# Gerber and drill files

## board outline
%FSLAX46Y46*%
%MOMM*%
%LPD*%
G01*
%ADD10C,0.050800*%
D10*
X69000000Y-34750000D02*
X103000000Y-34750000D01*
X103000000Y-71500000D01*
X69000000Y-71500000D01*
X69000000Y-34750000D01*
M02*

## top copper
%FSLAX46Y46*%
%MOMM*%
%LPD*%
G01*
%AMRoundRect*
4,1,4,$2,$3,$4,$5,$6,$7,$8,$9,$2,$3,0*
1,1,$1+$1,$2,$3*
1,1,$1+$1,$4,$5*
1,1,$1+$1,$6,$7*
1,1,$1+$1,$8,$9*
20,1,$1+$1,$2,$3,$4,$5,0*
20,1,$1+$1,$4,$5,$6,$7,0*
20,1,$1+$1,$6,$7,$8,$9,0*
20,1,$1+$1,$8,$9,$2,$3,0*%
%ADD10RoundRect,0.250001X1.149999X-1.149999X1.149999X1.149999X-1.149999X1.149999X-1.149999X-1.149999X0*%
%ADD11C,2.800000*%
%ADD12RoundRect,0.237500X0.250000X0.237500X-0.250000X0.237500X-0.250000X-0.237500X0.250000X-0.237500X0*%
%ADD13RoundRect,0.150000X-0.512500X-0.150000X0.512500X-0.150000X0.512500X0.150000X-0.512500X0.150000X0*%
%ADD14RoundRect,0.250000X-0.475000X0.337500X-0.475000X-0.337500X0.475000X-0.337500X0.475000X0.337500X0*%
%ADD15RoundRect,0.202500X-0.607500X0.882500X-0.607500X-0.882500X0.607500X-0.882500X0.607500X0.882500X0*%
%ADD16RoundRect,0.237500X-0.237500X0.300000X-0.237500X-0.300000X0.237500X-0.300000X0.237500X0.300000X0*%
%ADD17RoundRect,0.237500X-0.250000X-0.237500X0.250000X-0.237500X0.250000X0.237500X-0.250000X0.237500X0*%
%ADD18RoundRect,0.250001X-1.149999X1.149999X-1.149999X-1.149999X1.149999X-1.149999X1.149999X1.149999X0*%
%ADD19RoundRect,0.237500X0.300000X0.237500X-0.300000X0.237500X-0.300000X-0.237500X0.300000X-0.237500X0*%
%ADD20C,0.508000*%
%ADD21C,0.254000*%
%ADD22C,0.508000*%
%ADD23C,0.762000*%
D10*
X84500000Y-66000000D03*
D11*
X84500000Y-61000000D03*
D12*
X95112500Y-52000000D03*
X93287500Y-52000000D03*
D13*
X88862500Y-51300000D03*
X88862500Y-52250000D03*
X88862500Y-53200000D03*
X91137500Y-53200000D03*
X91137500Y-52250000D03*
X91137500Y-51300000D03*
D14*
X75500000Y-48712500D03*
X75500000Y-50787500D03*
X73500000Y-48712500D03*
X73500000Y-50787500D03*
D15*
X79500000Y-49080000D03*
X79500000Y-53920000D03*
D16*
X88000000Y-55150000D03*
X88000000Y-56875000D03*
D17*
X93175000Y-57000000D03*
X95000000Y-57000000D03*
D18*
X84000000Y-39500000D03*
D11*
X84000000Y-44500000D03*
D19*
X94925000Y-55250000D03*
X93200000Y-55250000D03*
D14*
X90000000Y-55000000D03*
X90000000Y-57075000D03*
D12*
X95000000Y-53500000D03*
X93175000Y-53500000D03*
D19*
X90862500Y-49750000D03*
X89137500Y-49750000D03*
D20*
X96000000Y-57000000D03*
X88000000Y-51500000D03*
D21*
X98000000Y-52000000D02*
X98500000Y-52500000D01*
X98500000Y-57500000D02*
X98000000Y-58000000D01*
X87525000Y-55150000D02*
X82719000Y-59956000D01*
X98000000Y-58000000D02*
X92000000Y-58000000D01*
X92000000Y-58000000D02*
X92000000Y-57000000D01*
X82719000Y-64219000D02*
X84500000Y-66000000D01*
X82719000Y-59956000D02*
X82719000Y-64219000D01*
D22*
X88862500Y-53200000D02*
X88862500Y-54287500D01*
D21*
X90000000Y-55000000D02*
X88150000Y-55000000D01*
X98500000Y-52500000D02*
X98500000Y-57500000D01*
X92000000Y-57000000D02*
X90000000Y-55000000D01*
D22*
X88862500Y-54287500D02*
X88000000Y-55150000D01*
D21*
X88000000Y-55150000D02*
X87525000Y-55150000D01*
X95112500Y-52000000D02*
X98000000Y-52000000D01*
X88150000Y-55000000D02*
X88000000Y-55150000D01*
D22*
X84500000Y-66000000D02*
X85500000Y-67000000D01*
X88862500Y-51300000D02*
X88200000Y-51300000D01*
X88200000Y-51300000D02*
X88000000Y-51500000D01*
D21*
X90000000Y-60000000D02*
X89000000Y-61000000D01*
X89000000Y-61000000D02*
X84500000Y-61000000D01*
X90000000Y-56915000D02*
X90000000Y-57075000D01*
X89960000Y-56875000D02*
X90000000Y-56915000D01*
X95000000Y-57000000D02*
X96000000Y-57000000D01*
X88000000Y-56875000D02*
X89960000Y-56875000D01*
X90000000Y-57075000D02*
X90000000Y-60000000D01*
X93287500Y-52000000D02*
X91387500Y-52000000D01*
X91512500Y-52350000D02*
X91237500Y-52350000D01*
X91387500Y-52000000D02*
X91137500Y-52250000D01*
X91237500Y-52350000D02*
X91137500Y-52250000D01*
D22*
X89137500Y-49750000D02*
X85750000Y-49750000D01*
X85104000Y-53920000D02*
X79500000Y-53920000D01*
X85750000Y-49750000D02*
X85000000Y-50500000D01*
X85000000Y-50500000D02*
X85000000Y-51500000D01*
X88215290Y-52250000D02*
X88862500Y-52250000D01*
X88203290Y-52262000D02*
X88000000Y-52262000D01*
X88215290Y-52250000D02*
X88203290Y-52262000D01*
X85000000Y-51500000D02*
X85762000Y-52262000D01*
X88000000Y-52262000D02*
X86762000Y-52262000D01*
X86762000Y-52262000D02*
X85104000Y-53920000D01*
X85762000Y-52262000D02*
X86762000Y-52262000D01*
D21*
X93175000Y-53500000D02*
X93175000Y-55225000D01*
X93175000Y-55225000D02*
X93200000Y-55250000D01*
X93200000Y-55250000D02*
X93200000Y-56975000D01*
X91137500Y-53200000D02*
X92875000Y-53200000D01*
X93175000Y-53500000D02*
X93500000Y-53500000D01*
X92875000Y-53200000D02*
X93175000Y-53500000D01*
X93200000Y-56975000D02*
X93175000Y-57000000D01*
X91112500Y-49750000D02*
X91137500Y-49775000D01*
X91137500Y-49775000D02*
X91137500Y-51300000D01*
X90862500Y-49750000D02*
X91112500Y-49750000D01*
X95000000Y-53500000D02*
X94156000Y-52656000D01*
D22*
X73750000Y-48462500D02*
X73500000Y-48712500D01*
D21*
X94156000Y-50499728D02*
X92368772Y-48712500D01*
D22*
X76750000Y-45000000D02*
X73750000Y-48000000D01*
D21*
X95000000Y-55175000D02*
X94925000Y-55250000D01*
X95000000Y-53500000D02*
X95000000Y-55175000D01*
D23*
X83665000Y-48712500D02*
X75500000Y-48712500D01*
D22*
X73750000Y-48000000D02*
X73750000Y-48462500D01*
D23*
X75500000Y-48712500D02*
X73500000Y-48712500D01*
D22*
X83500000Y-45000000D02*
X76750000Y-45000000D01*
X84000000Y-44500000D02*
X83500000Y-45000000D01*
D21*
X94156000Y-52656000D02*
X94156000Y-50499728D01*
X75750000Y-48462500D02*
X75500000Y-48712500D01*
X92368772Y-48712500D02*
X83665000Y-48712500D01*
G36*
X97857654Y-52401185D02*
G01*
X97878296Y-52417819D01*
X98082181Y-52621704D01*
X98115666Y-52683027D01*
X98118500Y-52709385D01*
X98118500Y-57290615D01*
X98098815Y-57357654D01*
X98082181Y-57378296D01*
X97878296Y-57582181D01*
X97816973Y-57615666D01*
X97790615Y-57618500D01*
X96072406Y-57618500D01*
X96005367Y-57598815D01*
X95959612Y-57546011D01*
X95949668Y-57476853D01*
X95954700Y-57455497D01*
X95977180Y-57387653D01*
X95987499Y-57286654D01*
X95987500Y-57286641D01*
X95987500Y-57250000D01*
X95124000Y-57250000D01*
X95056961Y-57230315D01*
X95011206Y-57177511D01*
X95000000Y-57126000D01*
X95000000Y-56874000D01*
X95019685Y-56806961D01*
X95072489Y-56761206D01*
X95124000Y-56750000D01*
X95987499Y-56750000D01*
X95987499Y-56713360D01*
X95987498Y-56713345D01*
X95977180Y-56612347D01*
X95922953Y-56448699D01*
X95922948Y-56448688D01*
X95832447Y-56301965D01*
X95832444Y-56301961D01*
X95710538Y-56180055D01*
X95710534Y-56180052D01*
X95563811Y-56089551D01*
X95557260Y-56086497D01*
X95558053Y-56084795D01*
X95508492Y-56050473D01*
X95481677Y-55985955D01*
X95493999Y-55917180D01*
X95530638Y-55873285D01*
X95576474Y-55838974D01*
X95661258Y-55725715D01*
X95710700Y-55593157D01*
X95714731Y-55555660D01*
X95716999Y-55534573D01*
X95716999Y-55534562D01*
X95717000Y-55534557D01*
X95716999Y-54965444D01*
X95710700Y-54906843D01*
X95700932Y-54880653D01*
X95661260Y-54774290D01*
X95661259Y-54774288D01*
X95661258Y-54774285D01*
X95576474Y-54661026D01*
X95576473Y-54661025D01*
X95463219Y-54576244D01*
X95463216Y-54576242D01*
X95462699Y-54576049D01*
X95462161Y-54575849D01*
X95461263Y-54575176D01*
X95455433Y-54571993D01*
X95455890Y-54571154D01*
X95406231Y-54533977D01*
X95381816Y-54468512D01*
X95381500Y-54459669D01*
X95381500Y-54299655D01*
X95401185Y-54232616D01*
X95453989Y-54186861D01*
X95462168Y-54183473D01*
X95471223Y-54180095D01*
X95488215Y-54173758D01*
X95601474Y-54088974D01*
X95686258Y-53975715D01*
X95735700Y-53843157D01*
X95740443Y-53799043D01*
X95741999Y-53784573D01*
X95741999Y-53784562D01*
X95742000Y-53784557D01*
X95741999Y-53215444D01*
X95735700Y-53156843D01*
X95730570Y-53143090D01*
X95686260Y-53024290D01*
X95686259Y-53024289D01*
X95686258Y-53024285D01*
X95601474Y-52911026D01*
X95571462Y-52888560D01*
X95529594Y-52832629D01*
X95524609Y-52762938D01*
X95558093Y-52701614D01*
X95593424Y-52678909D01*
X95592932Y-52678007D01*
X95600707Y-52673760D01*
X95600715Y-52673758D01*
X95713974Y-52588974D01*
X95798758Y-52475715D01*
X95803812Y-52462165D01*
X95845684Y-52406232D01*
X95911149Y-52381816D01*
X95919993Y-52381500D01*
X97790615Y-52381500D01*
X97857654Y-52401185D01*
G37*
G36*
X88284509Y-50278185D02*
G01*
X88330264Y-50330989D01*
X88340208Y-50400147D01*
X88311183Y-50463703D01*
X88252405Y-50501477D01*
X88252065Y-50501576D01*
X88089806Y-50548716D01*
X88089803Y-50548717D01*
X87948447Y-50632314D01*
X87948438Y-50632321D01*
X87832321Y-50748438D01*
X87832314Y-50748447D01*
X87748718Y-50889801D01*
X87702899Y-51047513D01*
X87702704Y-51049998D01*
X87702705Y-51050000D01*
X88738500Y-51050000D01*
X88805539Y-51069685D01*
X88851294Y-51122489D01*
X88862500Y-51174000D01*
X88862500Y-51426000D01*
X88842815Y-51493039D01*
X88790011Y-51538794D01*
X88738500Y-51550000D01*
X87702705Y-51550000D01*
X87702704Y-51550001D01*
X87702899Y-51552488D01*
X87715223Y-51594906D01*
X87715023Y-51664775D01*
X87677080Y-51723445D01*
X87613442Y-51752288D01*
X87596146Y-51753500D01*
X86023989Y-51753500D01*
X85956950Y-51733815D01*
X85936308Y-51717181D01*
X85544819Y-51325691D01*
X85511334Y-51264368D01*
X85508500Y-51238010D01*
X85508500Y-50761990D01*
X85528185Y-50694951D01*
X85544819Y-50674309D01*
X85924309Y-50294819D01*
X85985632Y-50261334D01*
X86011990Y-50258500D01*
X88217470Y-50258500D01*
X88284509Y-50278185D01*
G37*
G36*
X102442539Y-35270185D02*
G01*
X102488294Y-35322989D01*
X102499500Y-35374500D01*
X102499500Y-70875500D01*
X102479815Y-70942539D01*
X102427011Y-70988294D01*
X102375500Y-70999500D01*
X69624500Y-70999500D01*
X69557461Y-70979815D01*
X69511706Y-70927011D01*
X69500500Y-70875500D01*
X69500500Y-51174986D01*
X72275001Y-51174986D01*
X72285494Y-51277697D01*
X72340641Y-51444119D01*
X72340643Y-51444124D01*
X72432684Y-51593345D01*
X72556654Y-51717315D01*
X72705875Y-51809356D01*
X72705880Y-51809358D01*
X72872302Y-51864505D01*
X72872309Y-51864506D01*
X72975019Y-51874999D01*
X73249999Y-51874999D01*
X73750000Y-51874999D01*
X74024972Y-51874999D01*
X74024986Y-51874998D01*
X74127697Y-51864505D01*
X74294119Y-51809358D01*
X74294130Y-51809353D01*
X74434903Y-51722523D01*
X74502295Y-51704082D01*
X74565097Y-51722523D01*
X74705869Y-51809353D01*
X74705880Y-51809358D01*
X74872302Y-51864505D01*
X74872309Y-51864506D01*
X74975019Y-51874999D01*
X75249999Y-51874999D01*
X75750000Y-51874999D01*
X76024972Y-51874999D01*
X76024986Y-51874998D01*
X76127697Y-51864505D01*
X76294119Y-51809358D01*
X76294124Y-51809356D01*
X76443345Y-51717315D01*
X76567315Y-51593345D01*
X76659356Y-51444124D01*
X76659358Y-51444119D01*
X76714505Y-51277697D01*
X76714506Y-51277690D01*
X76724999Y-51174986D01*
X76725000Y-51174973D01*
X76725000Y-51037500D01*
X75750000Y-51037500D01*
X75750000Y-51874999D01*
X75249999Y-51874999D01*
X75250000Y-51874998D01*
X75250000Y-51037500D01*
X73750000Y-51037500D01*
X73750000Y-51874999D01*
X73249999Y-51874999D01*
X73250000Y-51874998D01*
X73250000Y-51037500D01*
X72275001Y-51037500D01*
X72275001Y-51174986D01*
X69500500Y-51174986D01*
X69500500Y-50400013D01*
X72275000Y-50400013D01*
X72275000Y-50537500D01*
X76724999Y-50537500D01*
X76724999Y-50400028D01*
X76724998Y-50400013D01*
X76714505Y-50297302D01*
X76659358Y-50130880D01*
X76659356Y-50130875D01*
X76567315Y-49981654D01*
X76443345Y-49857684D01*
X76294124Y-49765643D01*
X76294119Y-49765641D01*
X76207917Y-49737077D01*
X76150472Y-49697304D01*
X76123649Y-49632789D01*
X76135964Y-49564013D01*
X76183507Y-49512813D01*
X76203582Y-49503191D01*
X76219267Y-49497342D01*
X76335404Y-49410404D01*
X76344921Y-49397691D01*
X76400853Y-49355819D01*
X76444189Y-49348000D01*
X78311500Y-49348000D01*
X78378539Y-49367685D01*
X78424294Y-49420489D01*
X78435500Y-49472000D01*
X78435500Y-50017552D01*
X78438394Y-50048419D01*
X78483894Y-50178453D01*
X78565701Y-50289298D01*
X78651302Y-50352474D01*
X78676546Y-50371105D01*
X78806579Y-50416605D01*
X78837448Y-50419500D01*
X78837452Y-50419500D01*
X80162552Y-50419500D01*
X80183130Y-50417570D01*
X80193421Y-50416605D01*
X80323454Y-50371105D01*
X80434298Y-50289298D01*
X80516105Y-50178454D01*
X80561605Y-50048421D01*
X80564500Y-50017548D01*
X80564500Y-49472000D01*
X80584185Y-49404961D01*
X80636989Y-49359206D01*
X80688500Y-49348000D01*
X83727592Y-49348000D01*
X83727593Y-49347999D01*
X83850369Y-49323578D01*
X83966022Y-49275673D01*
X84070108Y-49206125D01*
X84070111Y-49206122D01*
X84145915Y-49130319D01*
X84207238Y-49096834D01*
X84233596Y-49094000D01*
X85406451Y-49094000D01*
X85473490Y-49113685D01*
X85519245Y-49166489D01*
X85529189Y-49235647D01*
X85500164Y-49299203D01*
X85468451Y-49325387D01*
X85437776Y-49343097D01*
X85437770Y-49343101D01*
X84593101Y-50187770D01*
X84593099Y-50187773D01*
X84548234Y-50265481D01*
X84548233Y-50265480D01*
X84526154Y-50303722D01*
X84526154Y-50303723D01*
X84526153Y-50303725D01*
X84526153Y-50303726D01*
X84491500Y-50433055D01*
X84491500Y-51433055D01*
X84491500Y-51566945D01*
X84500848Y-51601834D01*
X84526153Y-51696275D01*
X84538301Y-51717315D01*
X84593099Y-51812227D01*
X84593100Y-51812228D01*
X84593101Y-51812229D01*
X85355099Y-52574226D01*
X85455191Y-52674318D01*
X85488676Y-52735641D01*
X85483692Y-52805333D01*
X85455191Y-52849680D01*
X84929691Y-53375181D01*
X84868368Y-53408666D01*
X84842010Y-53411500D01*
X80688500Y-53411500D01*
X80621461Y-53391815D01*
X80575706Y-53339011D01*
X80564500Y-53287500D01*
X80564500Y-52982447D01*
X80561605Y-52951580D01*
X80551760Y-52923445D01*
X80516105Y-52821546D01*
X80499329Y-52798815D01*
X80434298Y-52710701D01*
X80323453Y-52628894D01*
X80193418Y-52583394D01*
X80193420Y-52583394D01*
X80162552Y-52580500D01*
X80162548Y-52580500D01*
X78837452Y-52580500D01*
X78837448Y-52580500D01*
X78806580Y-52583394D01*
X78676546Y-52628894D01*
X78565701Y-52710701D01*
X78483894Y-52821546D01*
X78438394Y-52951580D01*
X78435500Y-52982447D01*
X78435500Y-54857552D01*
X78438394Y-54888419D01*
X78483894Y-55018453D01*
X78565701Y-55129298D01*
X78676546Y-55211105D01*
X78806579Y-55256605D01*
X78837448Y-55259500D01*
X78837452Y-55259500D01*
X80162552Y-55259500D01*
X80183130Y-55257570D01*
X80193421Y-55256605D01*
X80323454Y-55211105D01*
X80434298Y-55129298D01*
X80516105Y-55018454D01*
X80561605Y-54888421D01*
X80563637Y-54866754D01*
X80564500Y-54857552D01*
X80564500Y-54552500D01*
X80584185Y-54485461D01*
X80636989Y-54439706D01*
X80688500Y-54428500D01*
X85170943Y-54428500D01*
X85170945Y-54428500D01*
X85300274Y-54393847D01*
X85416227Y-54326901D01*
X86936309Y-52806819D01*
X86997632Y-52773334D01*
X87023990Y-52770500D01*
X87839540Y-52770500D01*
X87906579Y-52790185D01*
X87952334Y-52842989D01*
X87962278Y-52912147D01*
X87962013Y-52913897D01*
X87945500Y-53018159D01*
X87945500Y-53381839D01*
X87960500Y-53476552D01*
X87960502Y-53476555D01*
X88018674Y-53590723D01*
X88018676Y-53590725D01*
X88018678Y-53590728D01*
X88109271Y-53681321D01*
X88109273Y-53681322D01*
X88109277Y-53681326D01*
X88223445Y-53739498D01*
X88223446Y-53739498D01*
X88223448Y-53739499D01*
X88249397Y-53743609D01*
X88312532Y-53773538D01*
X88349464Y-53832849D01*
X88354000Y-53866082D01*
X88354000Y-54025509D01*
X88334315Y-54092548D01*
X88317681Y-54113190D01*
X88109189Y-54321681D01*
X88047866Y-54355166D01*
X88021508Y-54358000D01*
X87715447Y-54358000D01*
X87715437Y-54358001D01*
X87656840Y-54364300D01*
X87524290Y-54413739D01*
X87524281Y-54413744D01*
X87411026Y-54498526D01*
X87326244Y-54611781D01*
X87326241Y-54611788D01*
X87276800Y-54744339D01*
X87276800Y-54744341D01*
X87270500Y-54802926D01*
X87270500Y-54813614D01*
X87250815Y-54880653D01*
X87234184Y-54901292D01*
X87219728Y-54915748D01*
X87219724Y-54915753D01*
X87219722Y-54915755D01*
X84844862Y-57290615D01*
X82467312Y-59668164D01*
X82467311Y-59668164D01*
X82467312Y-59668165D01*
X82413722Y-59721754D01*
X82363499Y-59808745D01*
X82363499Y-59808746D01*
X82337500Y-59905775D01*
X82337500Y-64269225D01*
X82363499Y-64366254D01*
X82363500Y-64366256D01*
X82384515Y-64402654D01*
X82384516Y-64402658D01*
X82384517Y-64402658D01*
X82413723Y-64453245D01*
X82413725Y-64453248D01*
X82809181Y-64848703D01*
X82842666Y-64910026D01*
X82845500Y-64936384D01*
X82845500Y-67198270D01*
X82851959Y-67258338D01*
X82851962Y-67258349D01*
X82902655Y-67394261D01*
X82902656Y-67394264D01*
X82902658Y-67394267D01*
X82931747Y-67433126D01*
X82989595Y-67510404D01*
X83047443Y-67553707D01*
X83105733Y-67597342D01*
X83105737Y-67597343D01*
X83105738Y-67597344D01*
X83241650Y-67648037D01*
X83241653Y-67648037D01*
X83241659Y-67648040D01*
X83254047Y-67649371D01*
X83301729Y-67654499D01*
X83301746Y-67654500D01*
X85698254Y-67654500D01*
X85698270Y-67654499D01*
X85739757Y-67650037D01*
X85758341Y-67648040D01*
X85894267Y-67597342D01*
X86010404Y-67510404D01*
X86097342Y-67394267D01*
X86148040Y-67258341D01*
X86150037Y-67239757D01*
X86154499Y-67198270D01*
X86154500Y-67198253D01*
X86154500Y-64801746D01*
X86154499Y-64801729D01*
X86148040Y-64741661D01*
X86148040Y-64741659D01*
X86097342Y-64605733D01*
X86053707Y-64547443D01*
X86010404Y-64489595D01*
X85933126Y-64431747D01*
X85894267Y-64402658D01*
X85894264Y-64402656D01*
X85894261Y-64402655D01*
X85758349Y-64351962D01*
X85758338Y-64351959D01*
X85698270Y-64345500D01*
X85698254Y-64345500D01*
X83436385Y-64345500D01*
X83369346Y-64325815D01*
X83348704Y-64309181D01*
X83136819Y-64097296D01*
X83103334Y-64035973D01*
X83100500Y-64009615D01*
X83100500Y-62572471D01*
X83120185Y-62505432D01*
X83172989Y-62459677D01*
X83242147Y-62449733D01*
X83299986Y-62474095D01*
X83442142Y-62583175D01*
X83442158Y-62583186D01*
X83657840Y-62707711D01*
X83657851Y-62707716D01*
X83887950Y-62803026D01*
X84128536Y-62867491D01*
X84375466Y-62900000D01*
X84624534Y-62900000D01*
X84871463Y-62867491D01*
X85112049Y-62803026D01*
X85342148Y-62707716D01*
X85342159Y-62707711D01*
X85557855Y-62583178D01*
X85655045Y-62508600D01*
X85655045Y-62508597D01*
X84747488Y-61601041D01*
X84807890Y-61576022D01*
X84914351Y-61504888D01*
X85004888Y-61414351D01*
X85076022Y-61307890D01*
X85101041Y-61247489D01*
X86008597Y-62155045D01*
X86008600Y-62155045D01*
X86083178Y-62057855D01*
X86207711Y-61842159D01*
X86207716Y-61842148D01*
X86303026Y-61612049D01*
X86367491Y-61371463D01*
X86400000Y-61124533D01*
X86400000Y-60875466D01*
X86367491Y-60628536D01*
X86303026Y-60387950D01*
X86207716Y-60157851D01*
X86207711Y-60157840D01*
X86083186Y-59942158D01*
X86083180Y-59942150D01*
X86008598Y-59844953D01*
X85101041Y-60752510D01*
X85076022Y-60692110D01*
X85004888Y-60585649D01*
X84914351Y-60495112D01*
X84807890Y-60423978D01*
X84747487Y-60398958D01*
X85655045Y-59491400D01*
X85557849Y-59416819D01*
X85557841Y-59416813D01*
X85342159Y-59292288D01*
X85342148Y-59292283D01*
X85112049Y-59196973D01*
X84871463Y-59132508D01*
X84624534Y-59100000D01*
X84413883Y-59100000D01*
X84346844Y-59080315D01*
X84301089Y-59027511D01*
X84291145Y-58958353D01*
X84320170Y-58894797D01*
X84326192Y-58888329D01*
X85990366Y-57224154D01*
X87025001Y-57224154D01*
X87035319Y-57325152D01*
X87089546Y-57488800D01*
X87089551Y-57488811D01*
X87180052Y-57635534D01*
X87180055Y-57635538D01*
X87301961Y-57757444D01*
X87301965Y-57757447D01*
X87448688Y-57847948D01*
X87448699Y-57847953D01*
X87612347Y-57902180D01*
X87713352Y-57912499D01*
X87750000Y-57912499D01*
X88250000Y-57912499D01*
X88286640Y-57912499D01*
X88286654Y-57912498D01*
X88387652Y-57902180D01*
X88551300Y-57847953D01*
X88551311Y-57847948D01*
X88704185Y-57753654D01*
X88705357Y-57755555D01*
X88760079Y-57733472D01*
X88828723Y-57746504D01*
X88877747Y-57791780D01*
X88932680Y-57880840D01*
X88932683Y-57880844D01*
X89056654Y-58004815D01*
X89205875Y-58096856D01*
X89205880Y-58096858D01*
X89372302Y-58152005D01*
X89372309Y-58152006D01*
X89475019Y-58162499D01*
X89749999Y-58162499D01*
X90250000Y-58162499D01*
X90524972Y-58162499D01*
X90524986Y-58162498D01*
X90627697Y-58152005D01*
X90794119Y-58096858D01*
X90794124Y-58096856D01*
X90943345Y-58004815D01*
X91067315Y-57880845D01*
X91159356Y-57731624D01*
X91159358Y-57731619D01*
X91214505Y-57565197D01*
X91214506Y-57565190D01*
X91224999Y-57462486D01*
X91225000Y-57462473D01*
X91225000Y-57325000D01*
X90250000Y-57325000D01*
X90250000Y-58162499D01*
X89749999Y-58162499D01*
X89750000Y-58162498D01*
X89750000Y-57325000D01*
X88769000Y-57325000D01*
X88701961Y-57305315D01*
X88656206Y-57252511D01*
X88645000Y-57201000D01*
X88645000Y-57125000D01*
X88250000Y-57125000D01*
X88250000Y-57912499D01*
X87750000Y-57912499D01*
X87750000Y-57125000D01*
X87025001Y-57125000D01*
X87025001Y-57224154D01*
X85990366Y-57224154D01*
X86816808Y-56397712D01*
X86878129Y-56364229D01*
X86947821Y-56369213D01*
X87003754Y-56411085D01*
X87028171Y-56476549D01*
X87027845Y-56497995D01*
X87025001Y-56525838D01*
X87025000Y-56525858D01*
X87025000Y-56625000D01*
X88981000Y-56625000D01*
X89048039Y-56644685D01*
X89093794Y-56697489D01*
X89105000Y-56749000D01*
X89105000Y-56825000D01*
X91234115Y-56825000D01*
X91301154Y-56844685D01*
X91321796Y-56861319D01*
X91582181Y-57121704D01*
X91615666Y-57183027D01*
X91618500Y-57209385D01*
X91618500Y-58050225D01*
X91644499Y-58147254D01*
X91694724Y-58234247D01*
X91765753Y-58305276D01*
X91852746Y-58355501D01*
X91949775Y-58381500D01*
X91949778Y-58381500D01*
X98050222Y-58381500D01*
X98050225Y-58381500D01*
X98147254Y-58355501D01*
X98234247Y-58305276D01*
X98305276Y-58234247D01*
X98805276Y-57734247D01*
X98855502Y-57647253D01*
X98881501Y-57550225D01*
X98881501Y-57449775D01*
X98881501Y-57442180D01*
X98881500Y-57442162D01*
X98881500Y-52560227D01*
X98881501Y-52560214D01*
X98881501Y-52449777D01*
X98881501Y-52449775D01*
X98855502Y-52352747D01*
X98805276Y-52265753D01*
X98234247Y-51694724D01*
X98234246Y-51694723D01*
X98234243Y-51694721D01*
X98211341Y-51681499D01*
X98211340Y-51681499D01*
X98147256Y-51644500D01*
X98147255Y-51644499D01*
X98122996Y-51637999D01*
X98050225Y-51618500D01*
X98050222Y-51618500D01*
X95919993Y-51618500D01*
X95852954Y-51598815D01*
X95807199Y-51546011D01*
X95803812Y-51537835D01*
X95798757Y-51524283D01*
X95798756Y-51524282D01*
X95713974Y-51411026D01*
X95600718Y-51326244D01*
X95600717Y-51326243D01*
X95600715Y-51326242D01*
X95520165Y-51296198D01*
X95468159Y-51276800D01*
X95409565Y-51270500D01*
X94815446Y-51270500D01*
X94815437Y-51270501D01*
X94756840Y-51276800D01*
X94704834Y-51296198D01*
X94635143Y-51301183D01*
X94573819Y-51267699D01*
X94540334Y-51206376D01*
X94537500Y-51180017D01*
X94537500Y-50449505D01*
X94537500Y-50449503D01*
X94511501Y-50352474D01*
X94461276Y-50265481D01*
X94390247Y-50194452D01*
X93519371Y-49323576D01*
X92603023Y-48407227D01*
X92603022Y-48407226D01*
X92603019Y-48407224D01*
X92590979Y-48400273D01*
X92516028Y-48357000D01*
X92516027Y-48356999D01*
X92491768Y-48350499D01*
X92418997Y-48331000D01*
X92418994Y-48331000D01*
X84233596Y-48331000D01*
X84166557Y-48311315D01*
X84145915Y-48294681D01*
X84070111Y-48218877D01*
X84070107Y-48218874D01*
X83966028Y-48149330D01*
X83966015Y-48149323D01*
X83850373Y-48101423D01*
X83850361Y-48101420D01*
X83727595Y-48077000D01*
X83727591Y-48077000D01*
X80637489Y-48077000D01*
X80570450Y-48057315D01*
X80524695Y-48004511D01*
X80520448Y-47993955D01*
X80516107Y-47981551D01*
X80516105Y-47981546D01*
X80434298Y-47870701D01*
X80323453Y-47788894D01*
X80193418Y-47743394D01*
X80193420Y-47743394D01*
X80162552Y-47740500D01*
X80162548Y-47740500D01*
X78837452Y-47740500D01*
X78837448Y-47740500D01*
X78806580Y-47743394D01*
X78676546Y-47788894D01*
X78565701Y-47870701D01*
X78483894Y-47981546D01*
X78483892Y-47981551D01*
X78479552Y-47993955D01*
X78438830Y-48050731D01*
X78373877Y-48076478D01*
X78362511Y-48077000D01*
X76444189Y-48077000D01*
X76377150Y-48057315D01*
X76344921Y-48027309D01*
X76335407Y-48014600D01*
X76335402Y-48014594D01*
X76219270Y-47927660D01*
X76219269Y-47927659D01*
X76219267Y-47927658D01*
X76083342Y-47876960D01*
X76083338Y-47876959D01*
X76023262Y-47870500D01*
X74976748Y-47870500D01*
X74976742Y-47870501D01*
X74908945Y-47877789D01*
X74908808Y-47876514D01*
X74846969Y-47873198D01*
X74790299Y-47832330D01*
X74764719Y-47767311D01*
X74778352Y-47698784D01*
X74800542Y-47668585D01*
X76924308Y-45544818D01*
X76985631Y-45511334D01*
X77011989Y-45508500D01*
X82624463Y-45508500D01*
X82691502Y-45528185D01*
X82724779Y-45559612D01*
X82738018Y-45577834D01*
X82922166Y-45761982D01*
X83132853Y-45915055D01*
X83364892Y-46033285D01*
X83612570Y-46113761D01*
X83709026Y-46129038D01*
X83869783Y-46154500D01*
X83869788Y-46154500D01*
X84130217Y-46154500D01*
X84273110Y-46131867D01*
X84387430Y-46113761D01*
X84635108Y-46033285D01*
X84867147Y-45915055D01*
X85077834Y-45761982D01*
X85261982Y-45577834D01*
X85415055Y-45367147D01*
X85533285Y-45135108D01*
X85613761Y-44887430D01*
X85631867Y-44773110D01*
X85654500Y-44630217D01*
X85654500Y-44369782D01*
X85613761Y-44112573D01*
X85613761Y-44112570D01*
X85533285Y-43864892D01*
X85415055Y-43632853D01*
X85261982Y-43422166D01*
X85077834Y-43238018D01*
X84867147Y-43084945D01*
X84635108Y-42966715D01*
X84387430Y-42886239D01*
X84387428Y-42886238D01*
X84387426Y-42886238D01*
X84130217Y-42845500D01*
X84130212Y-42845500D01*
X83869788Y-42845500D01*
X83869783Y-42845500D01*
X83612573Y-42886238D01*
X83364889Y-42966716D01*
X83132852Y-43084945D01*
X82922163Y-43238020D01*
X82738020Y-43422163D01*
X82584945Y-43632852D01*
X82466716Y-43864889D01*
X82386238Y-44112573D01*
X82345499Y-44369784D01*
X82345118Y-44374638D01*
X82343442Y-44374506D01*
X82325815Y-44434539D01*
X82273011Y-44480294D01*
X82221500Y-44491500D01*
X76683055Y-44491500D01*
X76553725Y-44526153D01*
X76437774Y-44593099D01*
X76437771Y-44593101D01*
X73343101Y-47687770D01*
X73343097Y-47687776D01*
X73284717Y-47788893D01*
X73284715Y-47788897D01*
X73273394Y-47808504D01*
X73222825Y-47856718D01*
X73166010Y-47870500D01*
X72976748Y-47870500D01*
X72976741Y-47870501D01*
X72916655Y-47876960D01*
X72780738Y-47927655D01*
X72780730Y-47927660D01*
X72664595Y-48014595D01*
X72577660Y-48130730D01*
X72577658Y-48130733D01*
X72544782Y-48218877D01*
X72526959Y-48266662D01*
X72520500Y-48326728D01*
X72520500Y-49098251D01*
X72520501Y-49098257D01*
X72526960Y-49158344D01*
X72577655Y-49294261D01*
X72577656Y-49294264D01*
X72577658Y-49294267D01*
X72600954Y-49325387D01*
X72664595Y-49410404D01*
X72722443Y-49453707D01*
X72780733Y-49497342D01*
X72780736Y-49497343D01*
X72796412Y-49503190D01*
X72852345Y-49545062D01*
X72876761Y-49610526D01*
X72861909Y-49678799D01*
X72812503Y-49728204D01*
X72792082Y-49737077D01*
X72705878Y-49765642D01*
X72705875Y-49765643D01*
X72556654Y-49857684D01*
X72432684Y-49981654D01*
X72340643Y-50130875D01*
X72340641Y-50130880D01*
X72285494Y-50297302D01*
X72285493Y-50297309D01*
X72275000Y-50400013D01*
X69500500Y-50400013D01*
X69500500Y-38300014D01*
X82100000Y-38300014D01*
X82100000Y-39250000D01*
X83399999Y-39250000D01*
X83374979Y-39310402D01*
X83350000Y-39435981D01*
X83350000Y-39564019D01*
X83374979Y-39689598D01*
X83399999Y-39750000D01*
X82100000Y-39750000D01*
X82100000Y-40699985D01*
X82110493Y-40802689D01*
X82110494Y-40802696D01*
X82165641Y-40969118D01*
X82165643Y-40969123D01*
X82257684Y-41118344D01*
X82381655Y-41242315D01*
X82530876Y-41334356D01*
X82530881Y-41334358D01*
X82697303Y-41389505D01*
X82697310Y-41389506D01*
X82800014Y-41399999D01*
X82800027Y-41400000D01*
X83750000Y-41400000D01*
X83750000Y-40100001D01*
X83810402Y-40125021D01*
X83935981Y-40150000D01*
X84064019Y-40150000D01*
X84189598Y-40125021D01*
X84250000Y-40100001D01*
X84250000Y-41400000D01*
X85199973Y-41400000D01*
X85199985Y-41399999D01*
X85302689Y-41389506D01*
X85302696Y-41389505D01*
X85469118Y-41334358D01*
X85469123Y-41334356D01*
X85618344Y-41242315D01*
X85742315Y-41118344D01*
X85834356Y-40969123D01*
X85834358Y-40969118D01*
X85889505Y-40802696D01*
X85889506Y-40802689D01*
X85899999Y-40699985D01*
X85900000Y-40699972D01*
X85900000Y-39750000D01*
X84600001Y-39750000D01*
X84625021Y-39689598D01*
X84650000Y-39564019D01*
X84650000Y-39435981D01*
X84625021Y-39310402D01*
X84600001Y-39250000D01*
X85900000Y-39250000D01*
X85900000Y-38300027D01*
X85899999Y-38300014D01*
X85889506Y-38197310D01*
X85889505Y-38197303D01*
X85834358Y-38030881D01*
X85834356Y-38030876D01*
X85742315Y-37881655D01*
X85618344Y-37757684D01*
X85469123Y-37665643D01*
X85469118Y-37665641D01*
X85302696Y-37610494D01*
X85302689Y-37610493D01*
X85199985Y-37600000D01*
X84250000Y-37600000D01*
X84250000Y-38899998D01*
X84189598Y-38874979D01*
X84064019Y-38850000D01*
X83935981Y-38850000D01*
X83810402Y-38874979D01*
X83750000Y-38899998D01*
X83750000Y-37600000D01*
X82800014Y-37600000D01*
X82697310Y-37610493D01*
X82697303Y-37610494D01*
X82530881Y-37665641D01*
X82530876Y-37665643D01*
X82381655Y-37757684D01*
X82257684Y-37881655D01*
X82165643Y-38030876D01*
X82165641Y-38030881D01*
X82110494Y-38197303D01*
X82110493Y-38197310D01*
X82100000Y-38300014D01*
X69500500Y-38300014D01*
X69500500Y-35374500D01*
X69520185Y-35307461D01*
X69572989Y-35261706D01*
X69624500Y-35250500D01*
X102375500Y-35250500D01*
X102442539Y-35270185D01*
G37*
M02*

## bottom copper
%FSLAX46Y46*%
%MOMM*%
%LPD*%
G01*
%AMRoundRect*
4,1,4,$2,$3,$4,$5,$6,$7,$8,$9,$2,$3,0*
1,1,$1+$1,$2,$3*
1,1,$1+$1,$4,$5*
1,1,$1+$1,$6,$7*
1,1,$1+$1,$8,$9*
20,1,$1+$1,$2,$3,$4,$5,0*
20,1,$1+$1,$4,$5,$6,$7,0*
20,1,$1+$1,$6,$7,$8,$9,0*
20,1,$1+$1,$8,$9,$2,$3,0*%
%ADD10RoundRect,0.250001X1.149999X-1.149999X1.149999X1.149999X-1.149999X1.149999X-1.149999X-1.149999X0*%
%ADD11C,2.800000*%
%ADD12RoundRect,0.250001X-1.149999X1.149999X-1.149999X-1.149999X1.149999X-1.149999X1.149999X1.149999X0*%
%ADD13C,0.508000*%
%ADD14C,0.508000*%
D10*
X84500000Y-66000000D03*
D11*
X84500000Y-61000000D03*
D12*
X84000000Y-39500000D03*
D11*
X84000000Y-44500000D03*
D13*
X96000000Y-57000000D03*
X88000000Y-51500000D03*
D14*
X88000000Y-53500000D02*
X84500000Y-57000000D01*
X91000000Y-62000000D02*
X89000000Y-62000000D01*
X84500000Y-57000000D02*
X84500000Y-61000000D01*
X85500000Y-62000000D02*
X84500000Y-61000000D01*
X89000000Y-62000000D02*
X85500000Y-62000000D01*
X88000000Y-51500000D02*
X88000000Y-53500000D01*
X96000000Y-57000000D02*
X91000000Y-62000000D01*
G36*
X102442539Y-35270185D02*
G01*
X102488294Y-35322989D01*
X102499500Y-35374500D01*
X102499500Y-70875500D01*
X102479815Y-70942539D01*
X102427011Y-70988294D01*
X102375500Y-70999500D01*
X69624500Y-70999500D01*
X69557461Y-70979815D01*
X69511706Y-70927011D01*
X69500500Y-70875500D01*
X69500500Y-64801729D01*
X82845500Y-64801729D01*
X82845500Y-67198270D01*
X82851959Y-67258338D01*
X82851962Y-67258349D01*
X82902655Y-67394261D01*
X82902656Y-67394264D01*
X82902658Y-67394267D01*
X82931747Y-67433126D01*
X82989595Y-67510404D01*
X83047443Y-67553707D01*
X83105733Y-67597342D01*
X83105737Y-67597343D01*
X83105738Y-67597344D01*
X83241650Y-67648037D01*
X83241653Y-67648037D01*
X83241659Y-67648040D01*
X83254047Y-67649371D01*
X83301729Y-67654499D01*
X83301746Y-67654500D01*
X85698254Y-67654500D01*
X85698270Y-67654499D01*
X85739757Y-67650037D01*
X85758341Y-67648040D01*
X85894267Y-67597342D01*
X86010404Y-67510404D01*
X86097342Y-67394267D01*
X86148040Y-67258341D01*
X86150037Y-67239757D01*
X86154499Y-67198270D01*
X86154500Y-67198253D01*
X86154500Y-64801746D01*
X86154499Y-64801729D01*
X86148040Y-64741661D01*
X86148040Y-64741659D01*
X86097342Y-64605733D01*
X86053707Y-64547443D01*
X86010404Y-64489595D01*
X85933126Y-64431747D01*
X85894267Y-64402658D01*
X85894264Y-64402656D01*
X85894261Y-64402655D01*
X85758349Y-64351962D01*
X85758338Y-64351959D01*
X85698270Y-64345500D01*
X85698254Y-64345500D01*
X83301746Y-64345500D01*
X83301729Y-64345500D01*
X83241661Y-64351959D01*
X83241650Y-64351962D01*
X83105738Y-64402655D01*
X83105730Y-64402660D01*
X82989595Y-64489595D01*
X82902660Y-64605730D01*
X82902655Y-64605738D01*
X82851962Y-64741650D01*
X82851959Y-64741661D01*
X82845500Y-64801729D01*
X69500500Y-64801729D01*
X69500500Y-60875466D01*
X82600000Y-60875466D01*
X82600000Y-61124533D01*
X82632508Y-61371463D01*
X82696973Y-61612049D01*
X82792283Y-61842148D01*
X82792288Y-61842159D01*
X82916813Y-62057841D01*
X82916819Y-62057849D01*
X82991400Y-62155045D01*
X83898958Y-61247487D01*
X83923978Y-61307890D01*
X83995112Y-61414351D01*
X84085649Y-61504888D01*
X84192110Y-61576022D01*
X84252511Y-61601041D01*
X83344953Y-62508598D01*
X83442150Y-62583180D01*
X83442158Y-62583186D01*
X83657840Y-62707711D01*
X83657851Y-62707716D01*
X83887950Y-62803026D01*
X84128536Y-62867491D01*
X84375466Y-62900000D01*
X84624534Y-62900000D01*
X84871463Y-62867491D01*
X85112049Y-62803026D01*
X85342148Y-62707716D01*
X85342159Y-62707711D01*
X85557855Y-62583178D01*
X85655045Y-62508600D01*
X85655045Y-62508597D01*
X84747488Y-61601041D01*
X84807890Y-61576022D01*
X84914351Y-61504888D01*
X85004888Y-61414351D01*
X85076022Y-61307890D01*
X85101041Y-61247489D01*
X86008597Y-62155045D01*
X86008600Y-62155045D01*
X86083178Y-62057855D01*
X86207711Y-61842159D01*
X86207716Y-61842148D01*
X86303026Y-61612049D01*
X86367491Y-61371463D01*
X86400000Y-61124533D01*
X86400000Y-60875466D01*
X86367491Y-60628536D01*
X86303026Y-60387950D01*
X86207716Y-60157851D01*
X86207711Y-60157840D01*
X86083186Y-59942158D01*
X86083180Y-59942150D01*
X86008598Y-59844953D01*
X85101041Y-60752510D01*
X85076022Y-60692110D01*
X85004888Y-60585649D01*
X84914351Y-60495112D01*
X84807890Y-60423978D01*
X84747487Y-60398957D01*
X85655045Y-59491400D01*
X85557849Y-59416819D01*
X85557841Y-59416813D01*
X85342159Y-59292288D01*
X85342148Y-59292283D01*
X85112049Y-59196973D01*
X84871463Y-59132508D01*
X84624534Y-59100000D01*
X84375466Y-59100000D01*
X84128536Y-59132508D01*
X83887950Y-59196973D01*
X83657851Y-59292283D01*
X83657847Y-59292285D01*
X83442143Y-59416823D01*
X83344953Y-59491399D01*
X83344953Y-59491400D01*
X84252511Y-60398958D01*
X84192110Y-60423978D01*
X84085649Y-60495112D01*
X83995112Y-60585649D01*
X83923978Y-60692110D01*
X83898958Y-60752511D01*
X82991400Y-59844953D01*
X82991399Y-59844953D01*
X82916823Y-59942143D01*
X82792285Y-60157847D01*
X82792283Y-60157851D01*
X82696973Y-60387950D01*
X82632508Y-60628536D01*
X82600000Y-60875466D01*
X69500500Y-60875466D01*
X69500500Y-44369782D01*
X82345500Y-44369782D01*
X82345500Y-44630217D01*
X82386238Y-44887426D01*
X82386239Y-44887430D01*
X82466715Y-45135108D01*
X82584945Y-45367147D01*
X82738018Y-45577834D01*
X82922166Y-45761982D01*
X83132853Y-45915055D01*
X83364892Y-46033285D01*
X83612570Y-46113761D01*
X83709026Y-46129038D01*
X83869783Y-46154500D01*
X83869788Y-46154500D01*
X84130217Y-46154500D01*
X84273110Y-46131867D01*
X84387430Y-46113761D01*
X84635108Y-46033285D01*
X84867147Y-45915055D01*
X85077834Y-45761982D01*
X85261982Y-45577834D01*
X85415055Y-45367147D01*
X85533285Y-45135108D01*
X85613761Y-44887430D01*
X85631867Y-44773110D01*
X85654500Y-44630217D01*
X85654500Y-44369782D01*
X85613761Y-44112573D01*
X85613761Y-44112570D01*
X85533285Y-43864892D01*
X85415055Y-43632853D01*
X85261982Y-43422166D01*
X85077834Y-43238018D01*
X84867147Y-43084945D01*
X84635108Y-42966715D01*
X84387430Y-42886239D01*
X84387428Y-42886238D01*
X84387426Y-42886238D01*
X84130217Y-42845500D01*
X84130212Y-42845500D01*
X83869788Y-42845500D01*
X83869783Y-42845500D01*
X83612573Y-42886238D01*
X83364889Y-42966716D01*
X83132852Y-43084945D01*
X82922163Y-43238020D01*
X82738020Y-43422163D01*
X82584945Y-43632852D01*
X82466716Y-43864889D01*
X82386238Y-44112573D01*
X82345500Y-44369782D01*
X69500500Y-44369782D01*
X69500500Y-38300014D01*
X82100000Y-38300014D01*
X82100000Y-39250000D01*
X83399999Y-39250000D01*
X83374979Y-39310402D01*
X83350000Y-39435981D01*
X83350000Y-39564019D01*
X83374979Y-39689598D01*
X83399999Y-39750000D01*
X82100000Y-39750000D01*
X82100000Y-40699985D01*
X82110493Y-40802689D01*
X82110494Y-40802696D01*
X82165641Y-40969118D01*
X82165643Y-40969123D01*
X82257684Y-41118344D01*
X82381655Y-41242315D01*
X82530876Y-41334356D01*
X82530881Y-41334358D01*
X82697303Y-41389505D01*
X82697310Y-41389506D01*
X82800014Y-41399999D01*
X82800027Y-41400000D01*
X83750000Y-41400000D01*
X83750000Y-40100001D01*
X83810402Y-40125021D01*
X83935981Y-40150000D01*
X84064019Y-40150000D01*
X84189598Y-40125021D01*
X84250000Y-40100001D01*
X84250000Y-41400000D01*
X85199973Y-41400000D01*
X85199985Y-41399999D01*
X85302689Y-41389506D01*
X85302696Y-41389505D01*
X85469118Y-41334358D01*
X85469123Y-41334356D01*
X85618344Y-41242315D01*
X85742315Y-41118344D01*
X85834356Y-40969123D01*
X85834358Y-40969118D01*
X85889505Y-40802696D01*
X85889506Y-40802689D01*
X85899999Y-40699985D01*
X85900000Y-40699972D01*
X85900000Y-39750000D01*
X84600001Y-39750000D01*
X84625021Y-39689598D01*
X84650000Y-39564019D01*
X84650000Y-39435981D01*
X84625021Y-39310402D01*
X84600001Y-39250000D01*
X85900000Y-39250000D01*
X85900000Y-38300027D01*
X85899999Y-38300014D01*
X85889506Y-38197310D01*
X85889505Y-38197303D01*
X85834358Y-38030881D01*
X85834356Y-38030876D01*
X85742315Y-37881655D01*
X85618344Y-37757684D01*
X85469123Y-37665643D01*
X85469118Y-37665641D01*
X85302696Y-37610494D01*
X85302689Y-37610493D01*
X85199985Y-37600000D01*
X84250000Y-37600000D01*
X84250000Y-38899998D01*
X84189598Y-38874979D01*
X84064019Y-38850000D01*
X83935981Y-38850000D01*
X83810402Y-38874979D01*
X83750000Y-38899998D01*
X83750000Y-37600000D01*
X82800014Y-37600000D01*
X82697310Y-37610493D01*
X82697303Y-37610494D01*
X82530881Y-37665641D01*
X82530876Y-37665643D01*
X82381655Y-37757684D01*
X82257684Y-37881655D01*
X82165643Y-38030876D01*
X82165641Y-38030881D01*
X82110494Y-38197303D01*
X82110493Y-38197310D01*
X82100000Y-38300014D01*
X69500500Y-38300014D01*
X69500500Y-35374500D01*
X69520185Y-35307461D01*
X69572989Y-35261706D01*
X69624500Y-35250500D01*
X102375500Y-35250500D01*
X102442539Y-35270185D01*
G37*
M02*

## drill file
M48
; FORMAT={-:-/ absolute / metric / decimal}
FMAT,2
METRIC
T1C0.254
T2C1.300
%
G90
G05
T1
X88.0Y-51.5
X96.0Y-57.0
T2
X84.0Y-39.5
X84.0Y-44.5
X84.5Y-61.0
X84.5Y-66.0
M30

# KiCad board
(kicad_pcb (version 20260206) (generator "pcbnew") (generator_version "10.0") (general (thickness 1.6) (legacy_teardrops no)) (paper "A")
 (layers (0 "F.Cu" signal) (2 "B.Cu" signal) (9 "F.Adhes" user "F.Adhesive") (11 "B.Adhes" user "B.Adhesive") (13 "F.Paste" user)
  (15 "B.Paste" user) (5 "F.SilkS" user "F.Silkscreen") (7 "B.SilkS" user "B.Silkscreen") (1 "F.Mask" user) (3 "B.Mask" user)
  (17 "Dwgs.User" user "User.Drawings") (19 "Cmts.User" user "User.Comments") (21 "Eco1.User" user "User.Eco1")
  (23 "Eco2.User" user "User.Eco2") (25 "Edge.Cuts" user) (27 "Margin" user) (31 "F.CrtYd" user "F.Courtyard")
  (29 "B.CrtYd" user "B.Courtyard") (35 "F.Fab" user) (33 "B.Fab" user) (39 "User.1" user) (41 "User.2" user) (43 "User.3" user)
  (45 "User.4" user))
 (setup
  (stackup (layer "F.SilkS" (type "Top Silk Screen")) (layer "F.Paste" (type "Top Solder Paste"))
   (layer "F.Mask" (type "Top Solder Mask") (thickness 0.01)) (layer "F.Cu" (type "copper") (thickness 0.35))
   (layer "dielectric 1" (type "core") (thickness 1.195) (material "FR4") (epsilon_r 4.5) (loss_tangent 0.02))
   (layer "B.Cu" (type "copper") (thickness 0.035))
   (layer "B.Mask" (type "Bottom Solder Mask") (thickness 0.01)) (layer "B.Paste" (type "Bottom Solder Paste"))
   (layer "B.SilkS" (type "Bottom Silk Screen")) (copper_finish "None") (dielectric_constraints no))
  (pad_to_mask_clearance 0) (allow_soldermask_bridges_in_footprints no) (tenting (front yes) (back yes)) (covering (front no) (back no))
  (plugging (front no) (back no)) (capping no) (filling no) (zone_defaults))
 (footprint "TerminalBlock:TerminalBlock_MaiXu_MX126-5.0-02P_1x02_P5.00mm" (layer "F.Cu") (at 84.5 66 90)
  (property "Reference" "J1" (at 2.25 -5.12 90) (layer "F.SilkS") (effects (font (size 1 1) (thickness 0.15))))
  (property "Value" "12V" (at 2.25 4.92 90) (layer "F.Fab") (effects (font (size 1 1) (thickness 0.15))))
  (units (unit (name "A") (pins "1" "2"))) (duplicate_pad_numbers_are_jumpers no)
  (pad "1" thru_hole roundrect (at 0 0 90) (size 2.8 2.8) (drill 1.3) (layers "*.Cu" "*.Mask") (remove_unused_layers no)
   (roundrect_rratio 0.089286) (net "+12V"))
  (pad "2" thru_hole circle (at 5 0 90) (size 2.8 2.8) (drill 1.3) (layers "*.Cu" "*.Mask") (remove_unused_layers no) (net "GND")))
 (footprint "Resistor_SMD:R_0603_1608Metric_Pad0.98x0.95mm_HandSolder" (layer "F.Cu") (at 94.2 52 180)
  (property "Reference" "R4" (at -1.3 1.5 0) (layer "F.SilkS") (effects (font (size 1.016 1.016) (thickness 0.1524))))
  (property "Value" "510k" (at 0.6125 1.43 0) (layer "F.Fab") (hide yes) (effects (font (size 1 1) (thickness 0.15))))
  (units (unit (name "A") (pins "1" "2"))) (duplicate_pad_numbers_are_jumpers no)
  (pad "1" smd roundrect (at -0.9125 0 180) (size 0.975 0.95) (layers "F.Cu" "F.Mask" "F.Paste") (roundrect_rratio 0.25) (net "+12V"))
  (pad "2" smd roundrect (at 0.9125 0 180) (size 0.975 0.95) (layers "F.Cu" "F.Mask" "F.Paste") (roundrect_rratio 0.25) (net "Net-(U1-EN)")))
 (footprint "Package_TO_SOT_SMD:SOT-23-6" (layer "F.Cu") (at 90 52.25)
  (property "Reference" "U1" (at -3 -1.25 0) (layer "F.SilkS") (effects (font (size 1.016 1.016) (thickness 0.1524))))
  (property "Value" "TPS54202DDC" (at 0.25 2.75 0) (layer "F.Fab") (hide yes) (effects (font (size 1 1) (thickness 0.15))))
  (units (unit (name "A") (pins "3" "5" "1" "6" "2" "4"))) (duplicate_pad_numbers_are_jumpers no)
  (pad "1" smd roundrect (at -1.1375 -0.95) (size 1.325 0.6) (layers "F.Cu" "F.Mask" "F.Paste") (roundrect_rratio 0.25) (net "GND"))
  (pad "2" smd roundrect (at -1.1375 0) (size 1.325 0.6) (layers "F.Cu" "F.Mask" "F.Paste") (roundrect_rratio 0.25) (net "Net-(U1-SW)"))
  (pad "3" smd roundrect (at -1.1375 0.95) (size 1.325 0.6) (layers "F.Cu" "F.Mask" "F.Paste") (roundrect_rratio 0.25) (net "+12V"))
  (pad "4" smd roundrect (at 1.1375 0.95) (size 1.325 0.6) (layers "F.Cu" "F.Mask" "F.Paste") (roundrect_rratio 0.25) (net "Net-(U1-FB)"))
  (pad "5" smd roundrect (at 1.1375 0) (size 1.325 0.6) (layers "F.Cu" "F.Mask" "F.Paste") (roundrect_rratio 0.25) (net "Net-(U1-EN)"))
  (pad "6" smd roundrect (at 1.1375 -0.95) (size 1.325 0.6) (layers "F.Cu" "F.Mask" "F.Paste") (roundrect_rratio 0.25) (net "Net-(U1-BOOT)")))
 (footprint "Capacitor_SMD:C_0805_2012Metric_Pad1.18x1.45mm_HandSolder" (layer "F.Cu") (at 75.5 49.75 -90)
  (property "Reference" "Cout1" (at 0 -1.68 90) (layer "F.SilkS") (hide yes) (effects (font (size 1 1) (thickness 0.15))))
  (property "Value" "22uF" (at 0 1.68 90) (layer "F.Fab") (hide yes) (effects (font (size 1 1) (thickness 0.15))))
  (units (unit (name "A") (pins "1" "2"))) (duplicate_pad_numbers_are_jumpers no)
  (pad "1" smd roundrect (at -1.0375 0 270) (size 1.175 1.45) (layers "F.Cu" "F.Mask" "F.Paste") (roundrect_rratio 0.212766) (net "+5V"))
  (pad "2" smd roundrect (at 1.0375 0 270) (size 1.175 1.45) (layers "F.Cu" "F.Mask" "F.Paste") (roundrect_rratio 0.212766) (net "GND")))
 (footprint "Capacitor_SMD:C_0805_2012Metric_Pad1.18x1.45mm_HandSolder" (layer "F.Cu") (at 73.5 49.75 -90)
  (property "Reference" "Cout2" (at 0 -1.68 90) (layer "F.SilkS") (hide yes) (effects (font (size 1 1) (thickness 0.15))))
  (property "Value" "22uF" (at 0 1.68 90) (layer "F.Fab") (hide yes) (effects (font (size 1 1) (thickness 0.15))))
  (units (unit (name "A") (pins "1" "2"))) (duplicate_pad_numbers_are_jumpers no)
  (pad "1" smd roundrect (at -1.0375 0 270) (size 1.175 1.45) (layers "F.Cu" "F.Mask" "F.Paste") (roundrect_rratio 0.212766) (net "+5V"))
  (pad "2" smd roundrect (at 1.0375 0 270) (size 1.175 1.45) (layers "F.Cu" "F.Mask" "F.Paste") (roundrect_rratio 0.212766) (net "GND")))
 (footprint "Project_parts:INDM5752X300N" (layer "F.Cu") (at 79.5 51.5 -90)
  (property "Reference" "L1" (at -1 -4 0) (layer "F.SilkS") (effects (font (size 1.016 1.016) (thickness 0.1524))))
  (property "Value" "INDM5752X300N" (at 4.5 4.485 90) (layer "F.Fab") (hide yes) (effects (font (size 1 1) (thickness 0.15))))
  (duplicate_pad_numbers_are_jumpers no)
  (pad "1" smd roundrect (at -2.42 0 270) (size 2.17 1.62) (layers "F.Cu" "F.Mask" "F.Paste") (roundrect_rratio 0.125) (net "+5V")
   (solder_mask_margin 0.102))
  (pad "2" smd roundrect (at 2.42 0 270) (size 2.17 1.62) (layers "F.Cu" "F.Mask" "F.Paste") (roundrect_rratio 0.125) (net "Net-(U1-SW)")
   (solder_mask_margin 0.102)))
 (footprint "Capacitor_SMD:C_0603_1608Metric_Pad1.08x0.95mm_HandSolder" (layer "F.Cu") (at 88 56.0125 -90)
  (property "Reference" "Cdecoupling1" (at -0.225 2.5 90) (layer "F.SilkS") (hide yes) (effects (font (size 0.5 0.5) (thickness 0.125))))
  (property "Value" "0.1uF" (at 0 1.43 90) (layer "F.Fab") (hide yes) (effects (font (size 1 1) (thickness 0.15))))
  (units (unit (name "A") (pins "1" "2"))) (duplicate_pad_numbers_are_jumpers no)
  (pad "1" smd roundrect (at -0.8625 0 270) (size 1.075 0.95) (layers "F.Cu" "F.Mask" "F.Paste") (roundrect_rratio 0.25) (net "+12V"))
  (pad "2" smd roundrect (at 0.8625 0 270) (size 1.075 0.95) (layers "F.Cu" "F.Mask" "F.Paste") (roundrect_rratio 0.25) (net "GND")))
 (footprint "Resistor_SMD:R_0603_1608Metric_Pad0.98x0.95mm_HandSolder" (layer "F.Cu") (at 94.0875 57)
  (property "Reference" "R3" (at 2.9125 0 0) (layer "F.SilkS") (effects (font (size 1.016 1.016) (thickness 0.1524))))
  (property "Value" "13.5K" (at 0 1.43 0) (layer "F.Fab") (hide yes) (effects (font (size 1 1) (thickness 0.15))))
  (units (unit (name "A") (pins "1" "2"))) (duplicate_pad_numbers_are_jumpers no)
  (pad "1" smd roundrect (at -0.9125 0) (size 0.975 0.95) (layers "F.Cu" "F.Mask" "F.Paste") (roundrect_rratio 0.25) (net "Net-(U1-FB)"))
  (pad "2" smd roundrect (at 0.9125 0) (size 0.975 0.95) (layers "F.Cu" "F.Mask" "F.Paste") (roundrect_rratio 0.25) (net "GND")))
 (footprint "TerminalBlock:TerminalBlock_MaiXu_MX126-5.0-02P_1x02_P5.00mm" (layer "F.Cu") (at 84 39.5 -90)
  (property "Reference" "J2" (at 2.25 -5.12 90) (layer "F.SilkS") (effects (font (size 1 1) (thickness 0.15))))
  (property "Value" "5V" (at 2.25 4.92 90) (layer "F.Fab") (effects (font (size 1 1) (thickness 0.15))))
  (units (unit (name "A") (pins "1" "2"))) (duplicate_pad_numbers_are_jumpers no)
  (pad "1" thru_hole roundrect (at 0 0 270) (size 2.8 2.8) (drill 1.3) (layers "*.Cu" "*.Mask") (remove_unused_layers no)
   (roundrect_rratio 0.089286) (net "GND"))
  (pad "2" thru_hole circle (at 5 0 270) (size 2.8 2.8) (drill 1.3) (layers "*.Cu" "*.Mask") (remove_unused_layers no) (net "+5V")))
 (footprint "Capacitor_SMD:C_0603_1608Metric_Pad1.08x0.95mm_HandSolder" (layer "F.Cu") (at 94.0625 55.25 180)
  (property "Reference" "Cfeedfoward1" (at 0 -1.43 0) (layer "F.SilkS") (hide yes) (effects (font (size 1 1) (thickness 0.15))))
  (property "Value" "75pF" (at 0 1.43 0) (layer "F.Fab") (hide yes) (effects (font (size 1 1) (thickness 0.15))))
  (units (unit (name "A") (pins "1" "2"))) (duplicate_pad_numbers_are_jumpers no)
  (pad "1" smd roundrect (at -0.8625 0 180) (size 1.075 0.95) (layers "F.Cu" "F.Mask" "F.Paste") (roundrect_rratio 0.25) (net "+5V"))
  (pad "2" smd roundrect (at 0.8625 0 180) (size 1.075 0.95) (layers "F.Cu" "F.Mask" "F.Paste") (roundrect_rratio 0.25) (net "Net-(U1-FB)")))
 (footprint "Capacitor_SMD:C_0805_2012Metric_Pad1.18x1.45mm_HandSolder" (layer "F.Cu") (at 90 56.0375 -90)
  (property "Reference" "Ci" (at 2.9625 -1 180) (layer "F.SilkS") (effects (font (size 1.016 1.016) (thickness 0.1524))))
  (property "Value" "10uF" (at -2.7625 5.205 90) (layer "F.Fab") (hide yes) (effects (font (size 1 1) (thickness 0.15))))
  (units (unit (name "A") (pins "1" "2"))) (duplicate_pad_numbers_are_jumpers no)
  (pad "1" smd roundrect (at -1.0375 0 270) (size 1.175 1.45) (layers "F.Cu" "F.Mask" "F.Paste") (roundrect_rratio 0.212766) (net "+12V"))
  (pad "2" smd roundrect (at 1.0375 0 270) (size 1.175 1.45) (layers "F.Cu" "F.Mask" "F.Paste") (roundrect_rratio 0.212766) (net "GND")))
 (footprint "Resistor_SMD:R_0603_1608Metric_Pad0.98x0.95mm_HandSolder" (layer "F.Cu") (at 94.0875 53.5 180)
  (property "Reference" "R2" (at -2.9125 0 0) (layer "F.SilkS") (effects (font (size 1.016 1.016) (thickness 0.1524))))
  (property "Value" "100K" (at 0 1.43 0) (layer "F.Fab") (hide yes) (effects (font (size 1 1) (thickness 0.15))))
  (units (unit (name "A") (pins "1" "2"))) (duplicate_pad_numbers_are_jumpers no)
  (pad "1" smd roundrect (at -0.9125 0 180) (size 0.975 0.95) (layers "F.Cu" "F.Mask" "F.Paste") (roundrect_rratio 0.25) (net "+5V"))
  (pad "2" smd roundrect (at 0.9125 0 180) (size 0.975 0.95) (layers "F.Cu" "F.Mask" "F.Paste") (roundrect_rratio 0.25) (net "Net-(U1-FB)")))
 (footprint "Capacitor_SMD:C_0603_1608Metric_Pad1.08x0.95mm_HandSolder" (layer "F.Cu") (at 90 49.75 180)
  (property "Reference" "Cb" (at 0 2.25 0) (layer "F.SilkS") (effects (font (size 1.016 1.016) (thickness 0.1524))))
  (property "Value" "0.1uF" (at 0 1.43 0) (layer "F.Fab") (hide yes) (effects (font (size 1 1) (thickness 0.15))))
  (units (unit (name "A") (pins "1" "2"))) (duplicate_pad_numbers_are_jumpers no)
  (pad "1" smd roundrect (at -0.8625 0 180) (size 1.075 0.95) (layers "F.Cu" "F.Mask" "F.Paste") (roundrect_rratio 0.25)
   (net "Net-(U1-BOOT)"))
  (pad "2" smd roundrect (at 0.8625 0 180) (size 1.075 0.95) (layers "F.Cu" "F.Mask" "F.Paste") (roundrect_rratio 0.25) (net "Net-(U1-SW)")))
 (gr_rect (start 69 34.75) (end 103 71.5) (stroke (width 0.0508) (type default)) (fill no) (layer "Edge.Cuts"))
 (segment (start 98 52) (end 98.5 52.5) (width 0.254) (layer "F.Cu") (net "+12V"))
 (segment (start 98.5 57.5) (end 98 58) (width 0.254) (layer "F.Cu") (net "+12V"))
 (segment (start 87.525 55.15) (end 82.719 59.956) (width 0.254) (layer "F.Cu") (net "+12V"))
 (segment (start 98 58) (end 92 58) (width 0.254) (layer "F.Cu") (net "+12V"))
 (segment (start 92 58) (end 92 57) (width 0.254) (layer "F.Cu") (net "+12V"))
 (segment (start 82.719 64.219) (end 84.5 66) (width 0.254) (layer "F.Cu") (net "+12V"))
 (segment (start 82.719 59.956) (end 82.719 64.219) (width 0.254) (layer "F.Cu") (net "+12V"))
 (segment (start 88.8625 53.2) (end 88.8625 54.2875) (width 0.508) (layer "F.Cu") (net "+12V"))
 (segment (start 90 55) (end 88.15 55) (width 0.254) (layer "F.Cu") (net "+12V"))
 (segment (start 98.5 52.5) (end 98.5 57.5) (width 0.254) (layer "F.Cu") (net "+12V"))
 (segment (start 92 57) (end 90 55) (width 0.254) (layer "F.Cu") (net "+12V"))
 (segment (start 88.8625 54.2875) (end 88 55.15) (width 0.508) (layer "F.Cu") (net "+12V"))
 (segment (start 88 55.15) (end 87.525 55.15) (width 0.254) (layer "F.Cu") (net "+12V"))
 (segment (start 95.1125 52) (end 98 52) (width 0.254) (layer "F.Cu") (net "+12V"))
 (segment (start 88.15 55) (end 88 55.15) (width 0.254) (layer "F.Cu") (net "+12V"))
 (segment (start 84.5 66) (end 85.5 67) (width 0.508) (layer "F.Cu") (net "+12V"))
 (segment (start 88.8625 51.3) (end 88.2 51.3) (width 0.508) (layer "F.Cu") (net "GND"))
 (segment (start 88.2 51.3) (end 88 51.5) (width 0.508) (layer "F.Cu") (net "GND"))
 (segment (start 90 60) (end 89 61) (width 0.254) (layer "F.Cu") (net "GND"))
 (segment (start 89 61) (end 84.5 61) (width 0.254) (layer "F.Cu") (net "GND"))
 (segment (start 90 56.915) (end 90 57.075) (width 0.254) (layer "F.Cu") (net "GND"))
 (segment (start 89.96 56.875) (end 90 56.915) (width 0.254) (layer "F.Cu") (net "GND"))
 (segment (start 95 57) (end 96 57) (width 0.254) (layer "F.Cu") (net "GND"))
 (segment (start 88 56.875) (end 89.96 56.875) (width 0.254) (layer "F.Cu") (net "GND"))
 (segment (start 90 57.075) (end 90 60) (width 0.254) (layer "F.Cu") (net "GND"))
 (via (at 96 57) (size 0.508) (drill 0.254) (layers "F.Cu" "B.Cu") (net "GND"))
 (via (at 88 51.5) (size 0.508) (drill 0.254) (layers "F.Cu" "B.Cu") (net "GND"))
 (segment (start 88 53.5) (end 84.5 57) (width 0.508) (layer "B.Cu") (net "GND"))
 (segment (start 91 62) (end 89 62) (width 0.508) (layer "B.Cu") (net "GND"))
 (segment (start 84.5 57) (end 84.5 61) (width 0.508) (layer "B.Cu") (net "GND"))
 (segment (start 85.5 62) (end 84.5 61) (width 0.508) (layer "B.Cu") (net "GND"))
 (segment (start 89 62) (end 85.5 62) (width 0.508) (layer "B.Cu") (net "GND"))
 (segment (start 88 51.5) (end 88 53.5) (width 0.508) (layer "B.Cu") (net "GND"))
 (segment (start 96 57) (end 91 62) (width 0.508) (layer "B.Cu") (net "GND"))
 (segment (start 93.2875 52) (end 91.3875 52) (width 0.254) (layer "F.Cu") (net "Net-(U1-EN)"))
 (segment (start 91.5125 52.35) (end 91.2375 52.35) (width 0.254) (layer "F.Cu") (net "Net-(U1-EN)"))
 (segment (start 91.3875 52) (end 91.1375 52.25) (width 0.254) (layer "F.Cu") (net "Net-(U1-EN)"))
 (segment (start 91.2375 52.35) (end 91.1375 52.25) (width 0.254) (layer "F.Cu") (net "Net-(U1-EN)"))
 (segment (start 89.1375 49.75) (end 85.75 49.75) (width 0.508) (layer "F.Cu") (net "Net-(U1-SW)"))
 (segment (start 85.104 53.92) (end 79.5 53.92) (width 0.508) (layer "F.Cu") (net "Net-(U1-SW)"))
 (segment (start 85.75 49.75) (end 85 50.5) (width 0.508) (layer "F.Cu") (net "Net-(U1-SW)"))
 (segment (start 85 50.5) (end 85 51.5) (width 0.508) (layer "F.Cu") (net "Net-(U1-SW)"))
 (segment (start 88.21529 52.25) (end 88.8625 52.25) (width 0.508) (layer "F.Cu") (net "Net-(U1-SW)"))
 (segment (start 88.20329 52.262) (end 88 52.262) (width 0.508) (layer "F.Cu") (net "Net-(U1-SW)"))
 (segment (start 88.21529 52.25) (end 88.20329 52.262) (width 0.508) (layer "F.Cu") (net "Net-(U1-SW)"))
 (segment (start 85 51.5) (end 85.762 52.262) (width 0.508) (layer "F.Cu") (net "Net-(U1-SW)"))
 (segment (start 88 52.262) (end 86.762 52.262) (width 0.508) (layer "F.Cu") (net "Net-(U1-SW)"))
 (segment (start 86.762 52.262) (end 85.104 53.92) (width 0.508) (layer "F.Cu") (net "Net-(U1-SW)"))
 (segment (start 85.762 52.262) (end 86.762 52.262) (width 0.508) (layer "F.Cu") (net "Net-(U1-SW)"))
 (segment (start 93.175 53.5) (end 93.175 55.225) (width 0.254) (layer "F.Cu") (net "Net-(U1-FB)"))
 (segment (start 93.175 55.225) (end 93.2 55.25) (width 0.254) (layer "F.Cu") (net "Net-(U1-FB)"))
 (segment (start 93.2 55.25) (end 93.2 56.975) (width 0.254) (layer "F.Cu") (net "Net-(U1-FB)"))
 (segment (start 91.1375 53.2) (end 92.875 53.2) (width 0.254) (layer "F.Cu") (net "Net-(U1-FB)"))
 (segment (start 93.175 53.5) (end 93.5 53.5) (width 0.254) (layer "F.Cu") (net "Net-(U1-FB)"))
 (segment (start 92.875 53.2) (end 93.175 53.5) (width 0.254) (layer "F.Cu") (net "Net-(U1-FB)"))
 (segment (start 93.2 56.975) (end 93.175 57) (width 0.254) (layer "F.Cu") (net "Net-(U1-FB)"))
 (segment (start 91.1125 49.75) (end 91.1375 49.775) (width 0.254) (layer "F.Cu") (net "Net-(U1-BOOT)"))
 (segment (start 91.1375 49.775) (end 91.1375 51.3) (width 0.254) (layer "F.Cu") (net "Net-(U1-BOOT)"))
 (segment (start 90.8625 49.75) (end 91.1125 49.75) (width 0.254) (layer "F.Cu") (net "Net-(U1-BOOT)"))
 (segment (start 95 53.5) (end 94.156 52.656) (width 0.254) (layer "F.Cu") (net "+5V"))
 (segment (start 73.75 48.4625) (end 73.5 48.7125) (width 0.508) (layer "F.Cu") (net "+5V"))
 (segment (start 94.156 50.499728) (end 92.368772 48.7125) (width 0.254) (layer "F.Cu") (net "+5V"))
 (segment (start 76.75 45) (end 73.75 48) (width 0.508) (layer "F.Cu") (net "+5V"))
 (segment (start 95 55.175) (end 94.925 55.25) (width 0.254) (layer "F.Cu") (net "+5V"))
 (segment (start 95 53.5) (end 95 55.175) (width 0.254) (layer "F.Cu") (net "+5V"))
 (segment (start 83.665 48.7125) (end 75.5 48.7125) (width 0.762) (layer "F.Cu") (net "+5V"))
 (segment (start 73.75 48) (end 73.75 48.4625) (width 0.508) (layer "F.Cu") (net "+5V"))
 (segment (start 75.5 48.7125) (end 73.5 48.7125) (width 0.762) (layer "F.Cu") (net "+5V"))
 (segment (start 83.5 45) (end 76.75 45) (width 0.508) (layer "F.Cu") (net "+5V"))
 (segment (start 84 44.5) (end 83.5 45) (width 0.508) (layer "F.Cu") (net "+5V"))
 (segment (start 94.156 52.656) (end 94.156 50.499728) (width 0.254) (layer "F.Cu") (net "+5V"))
 (segment (start 75.75 48.4625) (end 75.5 48.7125) (width 0.254) (layer "F.Cu") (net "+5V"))
 (segment (start 92.368772 48.7125) (end 83.665 48.7125) (width 0.254) (layer "F.Cu") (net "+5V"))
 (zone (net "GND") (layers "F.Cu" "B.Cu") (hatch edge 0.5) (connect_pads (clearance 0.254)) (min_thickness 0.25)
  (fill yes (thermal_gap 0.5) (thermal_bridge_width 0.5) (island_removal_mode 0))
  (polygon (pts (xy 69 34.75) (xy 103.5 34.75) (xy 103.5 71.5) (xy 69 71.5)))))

